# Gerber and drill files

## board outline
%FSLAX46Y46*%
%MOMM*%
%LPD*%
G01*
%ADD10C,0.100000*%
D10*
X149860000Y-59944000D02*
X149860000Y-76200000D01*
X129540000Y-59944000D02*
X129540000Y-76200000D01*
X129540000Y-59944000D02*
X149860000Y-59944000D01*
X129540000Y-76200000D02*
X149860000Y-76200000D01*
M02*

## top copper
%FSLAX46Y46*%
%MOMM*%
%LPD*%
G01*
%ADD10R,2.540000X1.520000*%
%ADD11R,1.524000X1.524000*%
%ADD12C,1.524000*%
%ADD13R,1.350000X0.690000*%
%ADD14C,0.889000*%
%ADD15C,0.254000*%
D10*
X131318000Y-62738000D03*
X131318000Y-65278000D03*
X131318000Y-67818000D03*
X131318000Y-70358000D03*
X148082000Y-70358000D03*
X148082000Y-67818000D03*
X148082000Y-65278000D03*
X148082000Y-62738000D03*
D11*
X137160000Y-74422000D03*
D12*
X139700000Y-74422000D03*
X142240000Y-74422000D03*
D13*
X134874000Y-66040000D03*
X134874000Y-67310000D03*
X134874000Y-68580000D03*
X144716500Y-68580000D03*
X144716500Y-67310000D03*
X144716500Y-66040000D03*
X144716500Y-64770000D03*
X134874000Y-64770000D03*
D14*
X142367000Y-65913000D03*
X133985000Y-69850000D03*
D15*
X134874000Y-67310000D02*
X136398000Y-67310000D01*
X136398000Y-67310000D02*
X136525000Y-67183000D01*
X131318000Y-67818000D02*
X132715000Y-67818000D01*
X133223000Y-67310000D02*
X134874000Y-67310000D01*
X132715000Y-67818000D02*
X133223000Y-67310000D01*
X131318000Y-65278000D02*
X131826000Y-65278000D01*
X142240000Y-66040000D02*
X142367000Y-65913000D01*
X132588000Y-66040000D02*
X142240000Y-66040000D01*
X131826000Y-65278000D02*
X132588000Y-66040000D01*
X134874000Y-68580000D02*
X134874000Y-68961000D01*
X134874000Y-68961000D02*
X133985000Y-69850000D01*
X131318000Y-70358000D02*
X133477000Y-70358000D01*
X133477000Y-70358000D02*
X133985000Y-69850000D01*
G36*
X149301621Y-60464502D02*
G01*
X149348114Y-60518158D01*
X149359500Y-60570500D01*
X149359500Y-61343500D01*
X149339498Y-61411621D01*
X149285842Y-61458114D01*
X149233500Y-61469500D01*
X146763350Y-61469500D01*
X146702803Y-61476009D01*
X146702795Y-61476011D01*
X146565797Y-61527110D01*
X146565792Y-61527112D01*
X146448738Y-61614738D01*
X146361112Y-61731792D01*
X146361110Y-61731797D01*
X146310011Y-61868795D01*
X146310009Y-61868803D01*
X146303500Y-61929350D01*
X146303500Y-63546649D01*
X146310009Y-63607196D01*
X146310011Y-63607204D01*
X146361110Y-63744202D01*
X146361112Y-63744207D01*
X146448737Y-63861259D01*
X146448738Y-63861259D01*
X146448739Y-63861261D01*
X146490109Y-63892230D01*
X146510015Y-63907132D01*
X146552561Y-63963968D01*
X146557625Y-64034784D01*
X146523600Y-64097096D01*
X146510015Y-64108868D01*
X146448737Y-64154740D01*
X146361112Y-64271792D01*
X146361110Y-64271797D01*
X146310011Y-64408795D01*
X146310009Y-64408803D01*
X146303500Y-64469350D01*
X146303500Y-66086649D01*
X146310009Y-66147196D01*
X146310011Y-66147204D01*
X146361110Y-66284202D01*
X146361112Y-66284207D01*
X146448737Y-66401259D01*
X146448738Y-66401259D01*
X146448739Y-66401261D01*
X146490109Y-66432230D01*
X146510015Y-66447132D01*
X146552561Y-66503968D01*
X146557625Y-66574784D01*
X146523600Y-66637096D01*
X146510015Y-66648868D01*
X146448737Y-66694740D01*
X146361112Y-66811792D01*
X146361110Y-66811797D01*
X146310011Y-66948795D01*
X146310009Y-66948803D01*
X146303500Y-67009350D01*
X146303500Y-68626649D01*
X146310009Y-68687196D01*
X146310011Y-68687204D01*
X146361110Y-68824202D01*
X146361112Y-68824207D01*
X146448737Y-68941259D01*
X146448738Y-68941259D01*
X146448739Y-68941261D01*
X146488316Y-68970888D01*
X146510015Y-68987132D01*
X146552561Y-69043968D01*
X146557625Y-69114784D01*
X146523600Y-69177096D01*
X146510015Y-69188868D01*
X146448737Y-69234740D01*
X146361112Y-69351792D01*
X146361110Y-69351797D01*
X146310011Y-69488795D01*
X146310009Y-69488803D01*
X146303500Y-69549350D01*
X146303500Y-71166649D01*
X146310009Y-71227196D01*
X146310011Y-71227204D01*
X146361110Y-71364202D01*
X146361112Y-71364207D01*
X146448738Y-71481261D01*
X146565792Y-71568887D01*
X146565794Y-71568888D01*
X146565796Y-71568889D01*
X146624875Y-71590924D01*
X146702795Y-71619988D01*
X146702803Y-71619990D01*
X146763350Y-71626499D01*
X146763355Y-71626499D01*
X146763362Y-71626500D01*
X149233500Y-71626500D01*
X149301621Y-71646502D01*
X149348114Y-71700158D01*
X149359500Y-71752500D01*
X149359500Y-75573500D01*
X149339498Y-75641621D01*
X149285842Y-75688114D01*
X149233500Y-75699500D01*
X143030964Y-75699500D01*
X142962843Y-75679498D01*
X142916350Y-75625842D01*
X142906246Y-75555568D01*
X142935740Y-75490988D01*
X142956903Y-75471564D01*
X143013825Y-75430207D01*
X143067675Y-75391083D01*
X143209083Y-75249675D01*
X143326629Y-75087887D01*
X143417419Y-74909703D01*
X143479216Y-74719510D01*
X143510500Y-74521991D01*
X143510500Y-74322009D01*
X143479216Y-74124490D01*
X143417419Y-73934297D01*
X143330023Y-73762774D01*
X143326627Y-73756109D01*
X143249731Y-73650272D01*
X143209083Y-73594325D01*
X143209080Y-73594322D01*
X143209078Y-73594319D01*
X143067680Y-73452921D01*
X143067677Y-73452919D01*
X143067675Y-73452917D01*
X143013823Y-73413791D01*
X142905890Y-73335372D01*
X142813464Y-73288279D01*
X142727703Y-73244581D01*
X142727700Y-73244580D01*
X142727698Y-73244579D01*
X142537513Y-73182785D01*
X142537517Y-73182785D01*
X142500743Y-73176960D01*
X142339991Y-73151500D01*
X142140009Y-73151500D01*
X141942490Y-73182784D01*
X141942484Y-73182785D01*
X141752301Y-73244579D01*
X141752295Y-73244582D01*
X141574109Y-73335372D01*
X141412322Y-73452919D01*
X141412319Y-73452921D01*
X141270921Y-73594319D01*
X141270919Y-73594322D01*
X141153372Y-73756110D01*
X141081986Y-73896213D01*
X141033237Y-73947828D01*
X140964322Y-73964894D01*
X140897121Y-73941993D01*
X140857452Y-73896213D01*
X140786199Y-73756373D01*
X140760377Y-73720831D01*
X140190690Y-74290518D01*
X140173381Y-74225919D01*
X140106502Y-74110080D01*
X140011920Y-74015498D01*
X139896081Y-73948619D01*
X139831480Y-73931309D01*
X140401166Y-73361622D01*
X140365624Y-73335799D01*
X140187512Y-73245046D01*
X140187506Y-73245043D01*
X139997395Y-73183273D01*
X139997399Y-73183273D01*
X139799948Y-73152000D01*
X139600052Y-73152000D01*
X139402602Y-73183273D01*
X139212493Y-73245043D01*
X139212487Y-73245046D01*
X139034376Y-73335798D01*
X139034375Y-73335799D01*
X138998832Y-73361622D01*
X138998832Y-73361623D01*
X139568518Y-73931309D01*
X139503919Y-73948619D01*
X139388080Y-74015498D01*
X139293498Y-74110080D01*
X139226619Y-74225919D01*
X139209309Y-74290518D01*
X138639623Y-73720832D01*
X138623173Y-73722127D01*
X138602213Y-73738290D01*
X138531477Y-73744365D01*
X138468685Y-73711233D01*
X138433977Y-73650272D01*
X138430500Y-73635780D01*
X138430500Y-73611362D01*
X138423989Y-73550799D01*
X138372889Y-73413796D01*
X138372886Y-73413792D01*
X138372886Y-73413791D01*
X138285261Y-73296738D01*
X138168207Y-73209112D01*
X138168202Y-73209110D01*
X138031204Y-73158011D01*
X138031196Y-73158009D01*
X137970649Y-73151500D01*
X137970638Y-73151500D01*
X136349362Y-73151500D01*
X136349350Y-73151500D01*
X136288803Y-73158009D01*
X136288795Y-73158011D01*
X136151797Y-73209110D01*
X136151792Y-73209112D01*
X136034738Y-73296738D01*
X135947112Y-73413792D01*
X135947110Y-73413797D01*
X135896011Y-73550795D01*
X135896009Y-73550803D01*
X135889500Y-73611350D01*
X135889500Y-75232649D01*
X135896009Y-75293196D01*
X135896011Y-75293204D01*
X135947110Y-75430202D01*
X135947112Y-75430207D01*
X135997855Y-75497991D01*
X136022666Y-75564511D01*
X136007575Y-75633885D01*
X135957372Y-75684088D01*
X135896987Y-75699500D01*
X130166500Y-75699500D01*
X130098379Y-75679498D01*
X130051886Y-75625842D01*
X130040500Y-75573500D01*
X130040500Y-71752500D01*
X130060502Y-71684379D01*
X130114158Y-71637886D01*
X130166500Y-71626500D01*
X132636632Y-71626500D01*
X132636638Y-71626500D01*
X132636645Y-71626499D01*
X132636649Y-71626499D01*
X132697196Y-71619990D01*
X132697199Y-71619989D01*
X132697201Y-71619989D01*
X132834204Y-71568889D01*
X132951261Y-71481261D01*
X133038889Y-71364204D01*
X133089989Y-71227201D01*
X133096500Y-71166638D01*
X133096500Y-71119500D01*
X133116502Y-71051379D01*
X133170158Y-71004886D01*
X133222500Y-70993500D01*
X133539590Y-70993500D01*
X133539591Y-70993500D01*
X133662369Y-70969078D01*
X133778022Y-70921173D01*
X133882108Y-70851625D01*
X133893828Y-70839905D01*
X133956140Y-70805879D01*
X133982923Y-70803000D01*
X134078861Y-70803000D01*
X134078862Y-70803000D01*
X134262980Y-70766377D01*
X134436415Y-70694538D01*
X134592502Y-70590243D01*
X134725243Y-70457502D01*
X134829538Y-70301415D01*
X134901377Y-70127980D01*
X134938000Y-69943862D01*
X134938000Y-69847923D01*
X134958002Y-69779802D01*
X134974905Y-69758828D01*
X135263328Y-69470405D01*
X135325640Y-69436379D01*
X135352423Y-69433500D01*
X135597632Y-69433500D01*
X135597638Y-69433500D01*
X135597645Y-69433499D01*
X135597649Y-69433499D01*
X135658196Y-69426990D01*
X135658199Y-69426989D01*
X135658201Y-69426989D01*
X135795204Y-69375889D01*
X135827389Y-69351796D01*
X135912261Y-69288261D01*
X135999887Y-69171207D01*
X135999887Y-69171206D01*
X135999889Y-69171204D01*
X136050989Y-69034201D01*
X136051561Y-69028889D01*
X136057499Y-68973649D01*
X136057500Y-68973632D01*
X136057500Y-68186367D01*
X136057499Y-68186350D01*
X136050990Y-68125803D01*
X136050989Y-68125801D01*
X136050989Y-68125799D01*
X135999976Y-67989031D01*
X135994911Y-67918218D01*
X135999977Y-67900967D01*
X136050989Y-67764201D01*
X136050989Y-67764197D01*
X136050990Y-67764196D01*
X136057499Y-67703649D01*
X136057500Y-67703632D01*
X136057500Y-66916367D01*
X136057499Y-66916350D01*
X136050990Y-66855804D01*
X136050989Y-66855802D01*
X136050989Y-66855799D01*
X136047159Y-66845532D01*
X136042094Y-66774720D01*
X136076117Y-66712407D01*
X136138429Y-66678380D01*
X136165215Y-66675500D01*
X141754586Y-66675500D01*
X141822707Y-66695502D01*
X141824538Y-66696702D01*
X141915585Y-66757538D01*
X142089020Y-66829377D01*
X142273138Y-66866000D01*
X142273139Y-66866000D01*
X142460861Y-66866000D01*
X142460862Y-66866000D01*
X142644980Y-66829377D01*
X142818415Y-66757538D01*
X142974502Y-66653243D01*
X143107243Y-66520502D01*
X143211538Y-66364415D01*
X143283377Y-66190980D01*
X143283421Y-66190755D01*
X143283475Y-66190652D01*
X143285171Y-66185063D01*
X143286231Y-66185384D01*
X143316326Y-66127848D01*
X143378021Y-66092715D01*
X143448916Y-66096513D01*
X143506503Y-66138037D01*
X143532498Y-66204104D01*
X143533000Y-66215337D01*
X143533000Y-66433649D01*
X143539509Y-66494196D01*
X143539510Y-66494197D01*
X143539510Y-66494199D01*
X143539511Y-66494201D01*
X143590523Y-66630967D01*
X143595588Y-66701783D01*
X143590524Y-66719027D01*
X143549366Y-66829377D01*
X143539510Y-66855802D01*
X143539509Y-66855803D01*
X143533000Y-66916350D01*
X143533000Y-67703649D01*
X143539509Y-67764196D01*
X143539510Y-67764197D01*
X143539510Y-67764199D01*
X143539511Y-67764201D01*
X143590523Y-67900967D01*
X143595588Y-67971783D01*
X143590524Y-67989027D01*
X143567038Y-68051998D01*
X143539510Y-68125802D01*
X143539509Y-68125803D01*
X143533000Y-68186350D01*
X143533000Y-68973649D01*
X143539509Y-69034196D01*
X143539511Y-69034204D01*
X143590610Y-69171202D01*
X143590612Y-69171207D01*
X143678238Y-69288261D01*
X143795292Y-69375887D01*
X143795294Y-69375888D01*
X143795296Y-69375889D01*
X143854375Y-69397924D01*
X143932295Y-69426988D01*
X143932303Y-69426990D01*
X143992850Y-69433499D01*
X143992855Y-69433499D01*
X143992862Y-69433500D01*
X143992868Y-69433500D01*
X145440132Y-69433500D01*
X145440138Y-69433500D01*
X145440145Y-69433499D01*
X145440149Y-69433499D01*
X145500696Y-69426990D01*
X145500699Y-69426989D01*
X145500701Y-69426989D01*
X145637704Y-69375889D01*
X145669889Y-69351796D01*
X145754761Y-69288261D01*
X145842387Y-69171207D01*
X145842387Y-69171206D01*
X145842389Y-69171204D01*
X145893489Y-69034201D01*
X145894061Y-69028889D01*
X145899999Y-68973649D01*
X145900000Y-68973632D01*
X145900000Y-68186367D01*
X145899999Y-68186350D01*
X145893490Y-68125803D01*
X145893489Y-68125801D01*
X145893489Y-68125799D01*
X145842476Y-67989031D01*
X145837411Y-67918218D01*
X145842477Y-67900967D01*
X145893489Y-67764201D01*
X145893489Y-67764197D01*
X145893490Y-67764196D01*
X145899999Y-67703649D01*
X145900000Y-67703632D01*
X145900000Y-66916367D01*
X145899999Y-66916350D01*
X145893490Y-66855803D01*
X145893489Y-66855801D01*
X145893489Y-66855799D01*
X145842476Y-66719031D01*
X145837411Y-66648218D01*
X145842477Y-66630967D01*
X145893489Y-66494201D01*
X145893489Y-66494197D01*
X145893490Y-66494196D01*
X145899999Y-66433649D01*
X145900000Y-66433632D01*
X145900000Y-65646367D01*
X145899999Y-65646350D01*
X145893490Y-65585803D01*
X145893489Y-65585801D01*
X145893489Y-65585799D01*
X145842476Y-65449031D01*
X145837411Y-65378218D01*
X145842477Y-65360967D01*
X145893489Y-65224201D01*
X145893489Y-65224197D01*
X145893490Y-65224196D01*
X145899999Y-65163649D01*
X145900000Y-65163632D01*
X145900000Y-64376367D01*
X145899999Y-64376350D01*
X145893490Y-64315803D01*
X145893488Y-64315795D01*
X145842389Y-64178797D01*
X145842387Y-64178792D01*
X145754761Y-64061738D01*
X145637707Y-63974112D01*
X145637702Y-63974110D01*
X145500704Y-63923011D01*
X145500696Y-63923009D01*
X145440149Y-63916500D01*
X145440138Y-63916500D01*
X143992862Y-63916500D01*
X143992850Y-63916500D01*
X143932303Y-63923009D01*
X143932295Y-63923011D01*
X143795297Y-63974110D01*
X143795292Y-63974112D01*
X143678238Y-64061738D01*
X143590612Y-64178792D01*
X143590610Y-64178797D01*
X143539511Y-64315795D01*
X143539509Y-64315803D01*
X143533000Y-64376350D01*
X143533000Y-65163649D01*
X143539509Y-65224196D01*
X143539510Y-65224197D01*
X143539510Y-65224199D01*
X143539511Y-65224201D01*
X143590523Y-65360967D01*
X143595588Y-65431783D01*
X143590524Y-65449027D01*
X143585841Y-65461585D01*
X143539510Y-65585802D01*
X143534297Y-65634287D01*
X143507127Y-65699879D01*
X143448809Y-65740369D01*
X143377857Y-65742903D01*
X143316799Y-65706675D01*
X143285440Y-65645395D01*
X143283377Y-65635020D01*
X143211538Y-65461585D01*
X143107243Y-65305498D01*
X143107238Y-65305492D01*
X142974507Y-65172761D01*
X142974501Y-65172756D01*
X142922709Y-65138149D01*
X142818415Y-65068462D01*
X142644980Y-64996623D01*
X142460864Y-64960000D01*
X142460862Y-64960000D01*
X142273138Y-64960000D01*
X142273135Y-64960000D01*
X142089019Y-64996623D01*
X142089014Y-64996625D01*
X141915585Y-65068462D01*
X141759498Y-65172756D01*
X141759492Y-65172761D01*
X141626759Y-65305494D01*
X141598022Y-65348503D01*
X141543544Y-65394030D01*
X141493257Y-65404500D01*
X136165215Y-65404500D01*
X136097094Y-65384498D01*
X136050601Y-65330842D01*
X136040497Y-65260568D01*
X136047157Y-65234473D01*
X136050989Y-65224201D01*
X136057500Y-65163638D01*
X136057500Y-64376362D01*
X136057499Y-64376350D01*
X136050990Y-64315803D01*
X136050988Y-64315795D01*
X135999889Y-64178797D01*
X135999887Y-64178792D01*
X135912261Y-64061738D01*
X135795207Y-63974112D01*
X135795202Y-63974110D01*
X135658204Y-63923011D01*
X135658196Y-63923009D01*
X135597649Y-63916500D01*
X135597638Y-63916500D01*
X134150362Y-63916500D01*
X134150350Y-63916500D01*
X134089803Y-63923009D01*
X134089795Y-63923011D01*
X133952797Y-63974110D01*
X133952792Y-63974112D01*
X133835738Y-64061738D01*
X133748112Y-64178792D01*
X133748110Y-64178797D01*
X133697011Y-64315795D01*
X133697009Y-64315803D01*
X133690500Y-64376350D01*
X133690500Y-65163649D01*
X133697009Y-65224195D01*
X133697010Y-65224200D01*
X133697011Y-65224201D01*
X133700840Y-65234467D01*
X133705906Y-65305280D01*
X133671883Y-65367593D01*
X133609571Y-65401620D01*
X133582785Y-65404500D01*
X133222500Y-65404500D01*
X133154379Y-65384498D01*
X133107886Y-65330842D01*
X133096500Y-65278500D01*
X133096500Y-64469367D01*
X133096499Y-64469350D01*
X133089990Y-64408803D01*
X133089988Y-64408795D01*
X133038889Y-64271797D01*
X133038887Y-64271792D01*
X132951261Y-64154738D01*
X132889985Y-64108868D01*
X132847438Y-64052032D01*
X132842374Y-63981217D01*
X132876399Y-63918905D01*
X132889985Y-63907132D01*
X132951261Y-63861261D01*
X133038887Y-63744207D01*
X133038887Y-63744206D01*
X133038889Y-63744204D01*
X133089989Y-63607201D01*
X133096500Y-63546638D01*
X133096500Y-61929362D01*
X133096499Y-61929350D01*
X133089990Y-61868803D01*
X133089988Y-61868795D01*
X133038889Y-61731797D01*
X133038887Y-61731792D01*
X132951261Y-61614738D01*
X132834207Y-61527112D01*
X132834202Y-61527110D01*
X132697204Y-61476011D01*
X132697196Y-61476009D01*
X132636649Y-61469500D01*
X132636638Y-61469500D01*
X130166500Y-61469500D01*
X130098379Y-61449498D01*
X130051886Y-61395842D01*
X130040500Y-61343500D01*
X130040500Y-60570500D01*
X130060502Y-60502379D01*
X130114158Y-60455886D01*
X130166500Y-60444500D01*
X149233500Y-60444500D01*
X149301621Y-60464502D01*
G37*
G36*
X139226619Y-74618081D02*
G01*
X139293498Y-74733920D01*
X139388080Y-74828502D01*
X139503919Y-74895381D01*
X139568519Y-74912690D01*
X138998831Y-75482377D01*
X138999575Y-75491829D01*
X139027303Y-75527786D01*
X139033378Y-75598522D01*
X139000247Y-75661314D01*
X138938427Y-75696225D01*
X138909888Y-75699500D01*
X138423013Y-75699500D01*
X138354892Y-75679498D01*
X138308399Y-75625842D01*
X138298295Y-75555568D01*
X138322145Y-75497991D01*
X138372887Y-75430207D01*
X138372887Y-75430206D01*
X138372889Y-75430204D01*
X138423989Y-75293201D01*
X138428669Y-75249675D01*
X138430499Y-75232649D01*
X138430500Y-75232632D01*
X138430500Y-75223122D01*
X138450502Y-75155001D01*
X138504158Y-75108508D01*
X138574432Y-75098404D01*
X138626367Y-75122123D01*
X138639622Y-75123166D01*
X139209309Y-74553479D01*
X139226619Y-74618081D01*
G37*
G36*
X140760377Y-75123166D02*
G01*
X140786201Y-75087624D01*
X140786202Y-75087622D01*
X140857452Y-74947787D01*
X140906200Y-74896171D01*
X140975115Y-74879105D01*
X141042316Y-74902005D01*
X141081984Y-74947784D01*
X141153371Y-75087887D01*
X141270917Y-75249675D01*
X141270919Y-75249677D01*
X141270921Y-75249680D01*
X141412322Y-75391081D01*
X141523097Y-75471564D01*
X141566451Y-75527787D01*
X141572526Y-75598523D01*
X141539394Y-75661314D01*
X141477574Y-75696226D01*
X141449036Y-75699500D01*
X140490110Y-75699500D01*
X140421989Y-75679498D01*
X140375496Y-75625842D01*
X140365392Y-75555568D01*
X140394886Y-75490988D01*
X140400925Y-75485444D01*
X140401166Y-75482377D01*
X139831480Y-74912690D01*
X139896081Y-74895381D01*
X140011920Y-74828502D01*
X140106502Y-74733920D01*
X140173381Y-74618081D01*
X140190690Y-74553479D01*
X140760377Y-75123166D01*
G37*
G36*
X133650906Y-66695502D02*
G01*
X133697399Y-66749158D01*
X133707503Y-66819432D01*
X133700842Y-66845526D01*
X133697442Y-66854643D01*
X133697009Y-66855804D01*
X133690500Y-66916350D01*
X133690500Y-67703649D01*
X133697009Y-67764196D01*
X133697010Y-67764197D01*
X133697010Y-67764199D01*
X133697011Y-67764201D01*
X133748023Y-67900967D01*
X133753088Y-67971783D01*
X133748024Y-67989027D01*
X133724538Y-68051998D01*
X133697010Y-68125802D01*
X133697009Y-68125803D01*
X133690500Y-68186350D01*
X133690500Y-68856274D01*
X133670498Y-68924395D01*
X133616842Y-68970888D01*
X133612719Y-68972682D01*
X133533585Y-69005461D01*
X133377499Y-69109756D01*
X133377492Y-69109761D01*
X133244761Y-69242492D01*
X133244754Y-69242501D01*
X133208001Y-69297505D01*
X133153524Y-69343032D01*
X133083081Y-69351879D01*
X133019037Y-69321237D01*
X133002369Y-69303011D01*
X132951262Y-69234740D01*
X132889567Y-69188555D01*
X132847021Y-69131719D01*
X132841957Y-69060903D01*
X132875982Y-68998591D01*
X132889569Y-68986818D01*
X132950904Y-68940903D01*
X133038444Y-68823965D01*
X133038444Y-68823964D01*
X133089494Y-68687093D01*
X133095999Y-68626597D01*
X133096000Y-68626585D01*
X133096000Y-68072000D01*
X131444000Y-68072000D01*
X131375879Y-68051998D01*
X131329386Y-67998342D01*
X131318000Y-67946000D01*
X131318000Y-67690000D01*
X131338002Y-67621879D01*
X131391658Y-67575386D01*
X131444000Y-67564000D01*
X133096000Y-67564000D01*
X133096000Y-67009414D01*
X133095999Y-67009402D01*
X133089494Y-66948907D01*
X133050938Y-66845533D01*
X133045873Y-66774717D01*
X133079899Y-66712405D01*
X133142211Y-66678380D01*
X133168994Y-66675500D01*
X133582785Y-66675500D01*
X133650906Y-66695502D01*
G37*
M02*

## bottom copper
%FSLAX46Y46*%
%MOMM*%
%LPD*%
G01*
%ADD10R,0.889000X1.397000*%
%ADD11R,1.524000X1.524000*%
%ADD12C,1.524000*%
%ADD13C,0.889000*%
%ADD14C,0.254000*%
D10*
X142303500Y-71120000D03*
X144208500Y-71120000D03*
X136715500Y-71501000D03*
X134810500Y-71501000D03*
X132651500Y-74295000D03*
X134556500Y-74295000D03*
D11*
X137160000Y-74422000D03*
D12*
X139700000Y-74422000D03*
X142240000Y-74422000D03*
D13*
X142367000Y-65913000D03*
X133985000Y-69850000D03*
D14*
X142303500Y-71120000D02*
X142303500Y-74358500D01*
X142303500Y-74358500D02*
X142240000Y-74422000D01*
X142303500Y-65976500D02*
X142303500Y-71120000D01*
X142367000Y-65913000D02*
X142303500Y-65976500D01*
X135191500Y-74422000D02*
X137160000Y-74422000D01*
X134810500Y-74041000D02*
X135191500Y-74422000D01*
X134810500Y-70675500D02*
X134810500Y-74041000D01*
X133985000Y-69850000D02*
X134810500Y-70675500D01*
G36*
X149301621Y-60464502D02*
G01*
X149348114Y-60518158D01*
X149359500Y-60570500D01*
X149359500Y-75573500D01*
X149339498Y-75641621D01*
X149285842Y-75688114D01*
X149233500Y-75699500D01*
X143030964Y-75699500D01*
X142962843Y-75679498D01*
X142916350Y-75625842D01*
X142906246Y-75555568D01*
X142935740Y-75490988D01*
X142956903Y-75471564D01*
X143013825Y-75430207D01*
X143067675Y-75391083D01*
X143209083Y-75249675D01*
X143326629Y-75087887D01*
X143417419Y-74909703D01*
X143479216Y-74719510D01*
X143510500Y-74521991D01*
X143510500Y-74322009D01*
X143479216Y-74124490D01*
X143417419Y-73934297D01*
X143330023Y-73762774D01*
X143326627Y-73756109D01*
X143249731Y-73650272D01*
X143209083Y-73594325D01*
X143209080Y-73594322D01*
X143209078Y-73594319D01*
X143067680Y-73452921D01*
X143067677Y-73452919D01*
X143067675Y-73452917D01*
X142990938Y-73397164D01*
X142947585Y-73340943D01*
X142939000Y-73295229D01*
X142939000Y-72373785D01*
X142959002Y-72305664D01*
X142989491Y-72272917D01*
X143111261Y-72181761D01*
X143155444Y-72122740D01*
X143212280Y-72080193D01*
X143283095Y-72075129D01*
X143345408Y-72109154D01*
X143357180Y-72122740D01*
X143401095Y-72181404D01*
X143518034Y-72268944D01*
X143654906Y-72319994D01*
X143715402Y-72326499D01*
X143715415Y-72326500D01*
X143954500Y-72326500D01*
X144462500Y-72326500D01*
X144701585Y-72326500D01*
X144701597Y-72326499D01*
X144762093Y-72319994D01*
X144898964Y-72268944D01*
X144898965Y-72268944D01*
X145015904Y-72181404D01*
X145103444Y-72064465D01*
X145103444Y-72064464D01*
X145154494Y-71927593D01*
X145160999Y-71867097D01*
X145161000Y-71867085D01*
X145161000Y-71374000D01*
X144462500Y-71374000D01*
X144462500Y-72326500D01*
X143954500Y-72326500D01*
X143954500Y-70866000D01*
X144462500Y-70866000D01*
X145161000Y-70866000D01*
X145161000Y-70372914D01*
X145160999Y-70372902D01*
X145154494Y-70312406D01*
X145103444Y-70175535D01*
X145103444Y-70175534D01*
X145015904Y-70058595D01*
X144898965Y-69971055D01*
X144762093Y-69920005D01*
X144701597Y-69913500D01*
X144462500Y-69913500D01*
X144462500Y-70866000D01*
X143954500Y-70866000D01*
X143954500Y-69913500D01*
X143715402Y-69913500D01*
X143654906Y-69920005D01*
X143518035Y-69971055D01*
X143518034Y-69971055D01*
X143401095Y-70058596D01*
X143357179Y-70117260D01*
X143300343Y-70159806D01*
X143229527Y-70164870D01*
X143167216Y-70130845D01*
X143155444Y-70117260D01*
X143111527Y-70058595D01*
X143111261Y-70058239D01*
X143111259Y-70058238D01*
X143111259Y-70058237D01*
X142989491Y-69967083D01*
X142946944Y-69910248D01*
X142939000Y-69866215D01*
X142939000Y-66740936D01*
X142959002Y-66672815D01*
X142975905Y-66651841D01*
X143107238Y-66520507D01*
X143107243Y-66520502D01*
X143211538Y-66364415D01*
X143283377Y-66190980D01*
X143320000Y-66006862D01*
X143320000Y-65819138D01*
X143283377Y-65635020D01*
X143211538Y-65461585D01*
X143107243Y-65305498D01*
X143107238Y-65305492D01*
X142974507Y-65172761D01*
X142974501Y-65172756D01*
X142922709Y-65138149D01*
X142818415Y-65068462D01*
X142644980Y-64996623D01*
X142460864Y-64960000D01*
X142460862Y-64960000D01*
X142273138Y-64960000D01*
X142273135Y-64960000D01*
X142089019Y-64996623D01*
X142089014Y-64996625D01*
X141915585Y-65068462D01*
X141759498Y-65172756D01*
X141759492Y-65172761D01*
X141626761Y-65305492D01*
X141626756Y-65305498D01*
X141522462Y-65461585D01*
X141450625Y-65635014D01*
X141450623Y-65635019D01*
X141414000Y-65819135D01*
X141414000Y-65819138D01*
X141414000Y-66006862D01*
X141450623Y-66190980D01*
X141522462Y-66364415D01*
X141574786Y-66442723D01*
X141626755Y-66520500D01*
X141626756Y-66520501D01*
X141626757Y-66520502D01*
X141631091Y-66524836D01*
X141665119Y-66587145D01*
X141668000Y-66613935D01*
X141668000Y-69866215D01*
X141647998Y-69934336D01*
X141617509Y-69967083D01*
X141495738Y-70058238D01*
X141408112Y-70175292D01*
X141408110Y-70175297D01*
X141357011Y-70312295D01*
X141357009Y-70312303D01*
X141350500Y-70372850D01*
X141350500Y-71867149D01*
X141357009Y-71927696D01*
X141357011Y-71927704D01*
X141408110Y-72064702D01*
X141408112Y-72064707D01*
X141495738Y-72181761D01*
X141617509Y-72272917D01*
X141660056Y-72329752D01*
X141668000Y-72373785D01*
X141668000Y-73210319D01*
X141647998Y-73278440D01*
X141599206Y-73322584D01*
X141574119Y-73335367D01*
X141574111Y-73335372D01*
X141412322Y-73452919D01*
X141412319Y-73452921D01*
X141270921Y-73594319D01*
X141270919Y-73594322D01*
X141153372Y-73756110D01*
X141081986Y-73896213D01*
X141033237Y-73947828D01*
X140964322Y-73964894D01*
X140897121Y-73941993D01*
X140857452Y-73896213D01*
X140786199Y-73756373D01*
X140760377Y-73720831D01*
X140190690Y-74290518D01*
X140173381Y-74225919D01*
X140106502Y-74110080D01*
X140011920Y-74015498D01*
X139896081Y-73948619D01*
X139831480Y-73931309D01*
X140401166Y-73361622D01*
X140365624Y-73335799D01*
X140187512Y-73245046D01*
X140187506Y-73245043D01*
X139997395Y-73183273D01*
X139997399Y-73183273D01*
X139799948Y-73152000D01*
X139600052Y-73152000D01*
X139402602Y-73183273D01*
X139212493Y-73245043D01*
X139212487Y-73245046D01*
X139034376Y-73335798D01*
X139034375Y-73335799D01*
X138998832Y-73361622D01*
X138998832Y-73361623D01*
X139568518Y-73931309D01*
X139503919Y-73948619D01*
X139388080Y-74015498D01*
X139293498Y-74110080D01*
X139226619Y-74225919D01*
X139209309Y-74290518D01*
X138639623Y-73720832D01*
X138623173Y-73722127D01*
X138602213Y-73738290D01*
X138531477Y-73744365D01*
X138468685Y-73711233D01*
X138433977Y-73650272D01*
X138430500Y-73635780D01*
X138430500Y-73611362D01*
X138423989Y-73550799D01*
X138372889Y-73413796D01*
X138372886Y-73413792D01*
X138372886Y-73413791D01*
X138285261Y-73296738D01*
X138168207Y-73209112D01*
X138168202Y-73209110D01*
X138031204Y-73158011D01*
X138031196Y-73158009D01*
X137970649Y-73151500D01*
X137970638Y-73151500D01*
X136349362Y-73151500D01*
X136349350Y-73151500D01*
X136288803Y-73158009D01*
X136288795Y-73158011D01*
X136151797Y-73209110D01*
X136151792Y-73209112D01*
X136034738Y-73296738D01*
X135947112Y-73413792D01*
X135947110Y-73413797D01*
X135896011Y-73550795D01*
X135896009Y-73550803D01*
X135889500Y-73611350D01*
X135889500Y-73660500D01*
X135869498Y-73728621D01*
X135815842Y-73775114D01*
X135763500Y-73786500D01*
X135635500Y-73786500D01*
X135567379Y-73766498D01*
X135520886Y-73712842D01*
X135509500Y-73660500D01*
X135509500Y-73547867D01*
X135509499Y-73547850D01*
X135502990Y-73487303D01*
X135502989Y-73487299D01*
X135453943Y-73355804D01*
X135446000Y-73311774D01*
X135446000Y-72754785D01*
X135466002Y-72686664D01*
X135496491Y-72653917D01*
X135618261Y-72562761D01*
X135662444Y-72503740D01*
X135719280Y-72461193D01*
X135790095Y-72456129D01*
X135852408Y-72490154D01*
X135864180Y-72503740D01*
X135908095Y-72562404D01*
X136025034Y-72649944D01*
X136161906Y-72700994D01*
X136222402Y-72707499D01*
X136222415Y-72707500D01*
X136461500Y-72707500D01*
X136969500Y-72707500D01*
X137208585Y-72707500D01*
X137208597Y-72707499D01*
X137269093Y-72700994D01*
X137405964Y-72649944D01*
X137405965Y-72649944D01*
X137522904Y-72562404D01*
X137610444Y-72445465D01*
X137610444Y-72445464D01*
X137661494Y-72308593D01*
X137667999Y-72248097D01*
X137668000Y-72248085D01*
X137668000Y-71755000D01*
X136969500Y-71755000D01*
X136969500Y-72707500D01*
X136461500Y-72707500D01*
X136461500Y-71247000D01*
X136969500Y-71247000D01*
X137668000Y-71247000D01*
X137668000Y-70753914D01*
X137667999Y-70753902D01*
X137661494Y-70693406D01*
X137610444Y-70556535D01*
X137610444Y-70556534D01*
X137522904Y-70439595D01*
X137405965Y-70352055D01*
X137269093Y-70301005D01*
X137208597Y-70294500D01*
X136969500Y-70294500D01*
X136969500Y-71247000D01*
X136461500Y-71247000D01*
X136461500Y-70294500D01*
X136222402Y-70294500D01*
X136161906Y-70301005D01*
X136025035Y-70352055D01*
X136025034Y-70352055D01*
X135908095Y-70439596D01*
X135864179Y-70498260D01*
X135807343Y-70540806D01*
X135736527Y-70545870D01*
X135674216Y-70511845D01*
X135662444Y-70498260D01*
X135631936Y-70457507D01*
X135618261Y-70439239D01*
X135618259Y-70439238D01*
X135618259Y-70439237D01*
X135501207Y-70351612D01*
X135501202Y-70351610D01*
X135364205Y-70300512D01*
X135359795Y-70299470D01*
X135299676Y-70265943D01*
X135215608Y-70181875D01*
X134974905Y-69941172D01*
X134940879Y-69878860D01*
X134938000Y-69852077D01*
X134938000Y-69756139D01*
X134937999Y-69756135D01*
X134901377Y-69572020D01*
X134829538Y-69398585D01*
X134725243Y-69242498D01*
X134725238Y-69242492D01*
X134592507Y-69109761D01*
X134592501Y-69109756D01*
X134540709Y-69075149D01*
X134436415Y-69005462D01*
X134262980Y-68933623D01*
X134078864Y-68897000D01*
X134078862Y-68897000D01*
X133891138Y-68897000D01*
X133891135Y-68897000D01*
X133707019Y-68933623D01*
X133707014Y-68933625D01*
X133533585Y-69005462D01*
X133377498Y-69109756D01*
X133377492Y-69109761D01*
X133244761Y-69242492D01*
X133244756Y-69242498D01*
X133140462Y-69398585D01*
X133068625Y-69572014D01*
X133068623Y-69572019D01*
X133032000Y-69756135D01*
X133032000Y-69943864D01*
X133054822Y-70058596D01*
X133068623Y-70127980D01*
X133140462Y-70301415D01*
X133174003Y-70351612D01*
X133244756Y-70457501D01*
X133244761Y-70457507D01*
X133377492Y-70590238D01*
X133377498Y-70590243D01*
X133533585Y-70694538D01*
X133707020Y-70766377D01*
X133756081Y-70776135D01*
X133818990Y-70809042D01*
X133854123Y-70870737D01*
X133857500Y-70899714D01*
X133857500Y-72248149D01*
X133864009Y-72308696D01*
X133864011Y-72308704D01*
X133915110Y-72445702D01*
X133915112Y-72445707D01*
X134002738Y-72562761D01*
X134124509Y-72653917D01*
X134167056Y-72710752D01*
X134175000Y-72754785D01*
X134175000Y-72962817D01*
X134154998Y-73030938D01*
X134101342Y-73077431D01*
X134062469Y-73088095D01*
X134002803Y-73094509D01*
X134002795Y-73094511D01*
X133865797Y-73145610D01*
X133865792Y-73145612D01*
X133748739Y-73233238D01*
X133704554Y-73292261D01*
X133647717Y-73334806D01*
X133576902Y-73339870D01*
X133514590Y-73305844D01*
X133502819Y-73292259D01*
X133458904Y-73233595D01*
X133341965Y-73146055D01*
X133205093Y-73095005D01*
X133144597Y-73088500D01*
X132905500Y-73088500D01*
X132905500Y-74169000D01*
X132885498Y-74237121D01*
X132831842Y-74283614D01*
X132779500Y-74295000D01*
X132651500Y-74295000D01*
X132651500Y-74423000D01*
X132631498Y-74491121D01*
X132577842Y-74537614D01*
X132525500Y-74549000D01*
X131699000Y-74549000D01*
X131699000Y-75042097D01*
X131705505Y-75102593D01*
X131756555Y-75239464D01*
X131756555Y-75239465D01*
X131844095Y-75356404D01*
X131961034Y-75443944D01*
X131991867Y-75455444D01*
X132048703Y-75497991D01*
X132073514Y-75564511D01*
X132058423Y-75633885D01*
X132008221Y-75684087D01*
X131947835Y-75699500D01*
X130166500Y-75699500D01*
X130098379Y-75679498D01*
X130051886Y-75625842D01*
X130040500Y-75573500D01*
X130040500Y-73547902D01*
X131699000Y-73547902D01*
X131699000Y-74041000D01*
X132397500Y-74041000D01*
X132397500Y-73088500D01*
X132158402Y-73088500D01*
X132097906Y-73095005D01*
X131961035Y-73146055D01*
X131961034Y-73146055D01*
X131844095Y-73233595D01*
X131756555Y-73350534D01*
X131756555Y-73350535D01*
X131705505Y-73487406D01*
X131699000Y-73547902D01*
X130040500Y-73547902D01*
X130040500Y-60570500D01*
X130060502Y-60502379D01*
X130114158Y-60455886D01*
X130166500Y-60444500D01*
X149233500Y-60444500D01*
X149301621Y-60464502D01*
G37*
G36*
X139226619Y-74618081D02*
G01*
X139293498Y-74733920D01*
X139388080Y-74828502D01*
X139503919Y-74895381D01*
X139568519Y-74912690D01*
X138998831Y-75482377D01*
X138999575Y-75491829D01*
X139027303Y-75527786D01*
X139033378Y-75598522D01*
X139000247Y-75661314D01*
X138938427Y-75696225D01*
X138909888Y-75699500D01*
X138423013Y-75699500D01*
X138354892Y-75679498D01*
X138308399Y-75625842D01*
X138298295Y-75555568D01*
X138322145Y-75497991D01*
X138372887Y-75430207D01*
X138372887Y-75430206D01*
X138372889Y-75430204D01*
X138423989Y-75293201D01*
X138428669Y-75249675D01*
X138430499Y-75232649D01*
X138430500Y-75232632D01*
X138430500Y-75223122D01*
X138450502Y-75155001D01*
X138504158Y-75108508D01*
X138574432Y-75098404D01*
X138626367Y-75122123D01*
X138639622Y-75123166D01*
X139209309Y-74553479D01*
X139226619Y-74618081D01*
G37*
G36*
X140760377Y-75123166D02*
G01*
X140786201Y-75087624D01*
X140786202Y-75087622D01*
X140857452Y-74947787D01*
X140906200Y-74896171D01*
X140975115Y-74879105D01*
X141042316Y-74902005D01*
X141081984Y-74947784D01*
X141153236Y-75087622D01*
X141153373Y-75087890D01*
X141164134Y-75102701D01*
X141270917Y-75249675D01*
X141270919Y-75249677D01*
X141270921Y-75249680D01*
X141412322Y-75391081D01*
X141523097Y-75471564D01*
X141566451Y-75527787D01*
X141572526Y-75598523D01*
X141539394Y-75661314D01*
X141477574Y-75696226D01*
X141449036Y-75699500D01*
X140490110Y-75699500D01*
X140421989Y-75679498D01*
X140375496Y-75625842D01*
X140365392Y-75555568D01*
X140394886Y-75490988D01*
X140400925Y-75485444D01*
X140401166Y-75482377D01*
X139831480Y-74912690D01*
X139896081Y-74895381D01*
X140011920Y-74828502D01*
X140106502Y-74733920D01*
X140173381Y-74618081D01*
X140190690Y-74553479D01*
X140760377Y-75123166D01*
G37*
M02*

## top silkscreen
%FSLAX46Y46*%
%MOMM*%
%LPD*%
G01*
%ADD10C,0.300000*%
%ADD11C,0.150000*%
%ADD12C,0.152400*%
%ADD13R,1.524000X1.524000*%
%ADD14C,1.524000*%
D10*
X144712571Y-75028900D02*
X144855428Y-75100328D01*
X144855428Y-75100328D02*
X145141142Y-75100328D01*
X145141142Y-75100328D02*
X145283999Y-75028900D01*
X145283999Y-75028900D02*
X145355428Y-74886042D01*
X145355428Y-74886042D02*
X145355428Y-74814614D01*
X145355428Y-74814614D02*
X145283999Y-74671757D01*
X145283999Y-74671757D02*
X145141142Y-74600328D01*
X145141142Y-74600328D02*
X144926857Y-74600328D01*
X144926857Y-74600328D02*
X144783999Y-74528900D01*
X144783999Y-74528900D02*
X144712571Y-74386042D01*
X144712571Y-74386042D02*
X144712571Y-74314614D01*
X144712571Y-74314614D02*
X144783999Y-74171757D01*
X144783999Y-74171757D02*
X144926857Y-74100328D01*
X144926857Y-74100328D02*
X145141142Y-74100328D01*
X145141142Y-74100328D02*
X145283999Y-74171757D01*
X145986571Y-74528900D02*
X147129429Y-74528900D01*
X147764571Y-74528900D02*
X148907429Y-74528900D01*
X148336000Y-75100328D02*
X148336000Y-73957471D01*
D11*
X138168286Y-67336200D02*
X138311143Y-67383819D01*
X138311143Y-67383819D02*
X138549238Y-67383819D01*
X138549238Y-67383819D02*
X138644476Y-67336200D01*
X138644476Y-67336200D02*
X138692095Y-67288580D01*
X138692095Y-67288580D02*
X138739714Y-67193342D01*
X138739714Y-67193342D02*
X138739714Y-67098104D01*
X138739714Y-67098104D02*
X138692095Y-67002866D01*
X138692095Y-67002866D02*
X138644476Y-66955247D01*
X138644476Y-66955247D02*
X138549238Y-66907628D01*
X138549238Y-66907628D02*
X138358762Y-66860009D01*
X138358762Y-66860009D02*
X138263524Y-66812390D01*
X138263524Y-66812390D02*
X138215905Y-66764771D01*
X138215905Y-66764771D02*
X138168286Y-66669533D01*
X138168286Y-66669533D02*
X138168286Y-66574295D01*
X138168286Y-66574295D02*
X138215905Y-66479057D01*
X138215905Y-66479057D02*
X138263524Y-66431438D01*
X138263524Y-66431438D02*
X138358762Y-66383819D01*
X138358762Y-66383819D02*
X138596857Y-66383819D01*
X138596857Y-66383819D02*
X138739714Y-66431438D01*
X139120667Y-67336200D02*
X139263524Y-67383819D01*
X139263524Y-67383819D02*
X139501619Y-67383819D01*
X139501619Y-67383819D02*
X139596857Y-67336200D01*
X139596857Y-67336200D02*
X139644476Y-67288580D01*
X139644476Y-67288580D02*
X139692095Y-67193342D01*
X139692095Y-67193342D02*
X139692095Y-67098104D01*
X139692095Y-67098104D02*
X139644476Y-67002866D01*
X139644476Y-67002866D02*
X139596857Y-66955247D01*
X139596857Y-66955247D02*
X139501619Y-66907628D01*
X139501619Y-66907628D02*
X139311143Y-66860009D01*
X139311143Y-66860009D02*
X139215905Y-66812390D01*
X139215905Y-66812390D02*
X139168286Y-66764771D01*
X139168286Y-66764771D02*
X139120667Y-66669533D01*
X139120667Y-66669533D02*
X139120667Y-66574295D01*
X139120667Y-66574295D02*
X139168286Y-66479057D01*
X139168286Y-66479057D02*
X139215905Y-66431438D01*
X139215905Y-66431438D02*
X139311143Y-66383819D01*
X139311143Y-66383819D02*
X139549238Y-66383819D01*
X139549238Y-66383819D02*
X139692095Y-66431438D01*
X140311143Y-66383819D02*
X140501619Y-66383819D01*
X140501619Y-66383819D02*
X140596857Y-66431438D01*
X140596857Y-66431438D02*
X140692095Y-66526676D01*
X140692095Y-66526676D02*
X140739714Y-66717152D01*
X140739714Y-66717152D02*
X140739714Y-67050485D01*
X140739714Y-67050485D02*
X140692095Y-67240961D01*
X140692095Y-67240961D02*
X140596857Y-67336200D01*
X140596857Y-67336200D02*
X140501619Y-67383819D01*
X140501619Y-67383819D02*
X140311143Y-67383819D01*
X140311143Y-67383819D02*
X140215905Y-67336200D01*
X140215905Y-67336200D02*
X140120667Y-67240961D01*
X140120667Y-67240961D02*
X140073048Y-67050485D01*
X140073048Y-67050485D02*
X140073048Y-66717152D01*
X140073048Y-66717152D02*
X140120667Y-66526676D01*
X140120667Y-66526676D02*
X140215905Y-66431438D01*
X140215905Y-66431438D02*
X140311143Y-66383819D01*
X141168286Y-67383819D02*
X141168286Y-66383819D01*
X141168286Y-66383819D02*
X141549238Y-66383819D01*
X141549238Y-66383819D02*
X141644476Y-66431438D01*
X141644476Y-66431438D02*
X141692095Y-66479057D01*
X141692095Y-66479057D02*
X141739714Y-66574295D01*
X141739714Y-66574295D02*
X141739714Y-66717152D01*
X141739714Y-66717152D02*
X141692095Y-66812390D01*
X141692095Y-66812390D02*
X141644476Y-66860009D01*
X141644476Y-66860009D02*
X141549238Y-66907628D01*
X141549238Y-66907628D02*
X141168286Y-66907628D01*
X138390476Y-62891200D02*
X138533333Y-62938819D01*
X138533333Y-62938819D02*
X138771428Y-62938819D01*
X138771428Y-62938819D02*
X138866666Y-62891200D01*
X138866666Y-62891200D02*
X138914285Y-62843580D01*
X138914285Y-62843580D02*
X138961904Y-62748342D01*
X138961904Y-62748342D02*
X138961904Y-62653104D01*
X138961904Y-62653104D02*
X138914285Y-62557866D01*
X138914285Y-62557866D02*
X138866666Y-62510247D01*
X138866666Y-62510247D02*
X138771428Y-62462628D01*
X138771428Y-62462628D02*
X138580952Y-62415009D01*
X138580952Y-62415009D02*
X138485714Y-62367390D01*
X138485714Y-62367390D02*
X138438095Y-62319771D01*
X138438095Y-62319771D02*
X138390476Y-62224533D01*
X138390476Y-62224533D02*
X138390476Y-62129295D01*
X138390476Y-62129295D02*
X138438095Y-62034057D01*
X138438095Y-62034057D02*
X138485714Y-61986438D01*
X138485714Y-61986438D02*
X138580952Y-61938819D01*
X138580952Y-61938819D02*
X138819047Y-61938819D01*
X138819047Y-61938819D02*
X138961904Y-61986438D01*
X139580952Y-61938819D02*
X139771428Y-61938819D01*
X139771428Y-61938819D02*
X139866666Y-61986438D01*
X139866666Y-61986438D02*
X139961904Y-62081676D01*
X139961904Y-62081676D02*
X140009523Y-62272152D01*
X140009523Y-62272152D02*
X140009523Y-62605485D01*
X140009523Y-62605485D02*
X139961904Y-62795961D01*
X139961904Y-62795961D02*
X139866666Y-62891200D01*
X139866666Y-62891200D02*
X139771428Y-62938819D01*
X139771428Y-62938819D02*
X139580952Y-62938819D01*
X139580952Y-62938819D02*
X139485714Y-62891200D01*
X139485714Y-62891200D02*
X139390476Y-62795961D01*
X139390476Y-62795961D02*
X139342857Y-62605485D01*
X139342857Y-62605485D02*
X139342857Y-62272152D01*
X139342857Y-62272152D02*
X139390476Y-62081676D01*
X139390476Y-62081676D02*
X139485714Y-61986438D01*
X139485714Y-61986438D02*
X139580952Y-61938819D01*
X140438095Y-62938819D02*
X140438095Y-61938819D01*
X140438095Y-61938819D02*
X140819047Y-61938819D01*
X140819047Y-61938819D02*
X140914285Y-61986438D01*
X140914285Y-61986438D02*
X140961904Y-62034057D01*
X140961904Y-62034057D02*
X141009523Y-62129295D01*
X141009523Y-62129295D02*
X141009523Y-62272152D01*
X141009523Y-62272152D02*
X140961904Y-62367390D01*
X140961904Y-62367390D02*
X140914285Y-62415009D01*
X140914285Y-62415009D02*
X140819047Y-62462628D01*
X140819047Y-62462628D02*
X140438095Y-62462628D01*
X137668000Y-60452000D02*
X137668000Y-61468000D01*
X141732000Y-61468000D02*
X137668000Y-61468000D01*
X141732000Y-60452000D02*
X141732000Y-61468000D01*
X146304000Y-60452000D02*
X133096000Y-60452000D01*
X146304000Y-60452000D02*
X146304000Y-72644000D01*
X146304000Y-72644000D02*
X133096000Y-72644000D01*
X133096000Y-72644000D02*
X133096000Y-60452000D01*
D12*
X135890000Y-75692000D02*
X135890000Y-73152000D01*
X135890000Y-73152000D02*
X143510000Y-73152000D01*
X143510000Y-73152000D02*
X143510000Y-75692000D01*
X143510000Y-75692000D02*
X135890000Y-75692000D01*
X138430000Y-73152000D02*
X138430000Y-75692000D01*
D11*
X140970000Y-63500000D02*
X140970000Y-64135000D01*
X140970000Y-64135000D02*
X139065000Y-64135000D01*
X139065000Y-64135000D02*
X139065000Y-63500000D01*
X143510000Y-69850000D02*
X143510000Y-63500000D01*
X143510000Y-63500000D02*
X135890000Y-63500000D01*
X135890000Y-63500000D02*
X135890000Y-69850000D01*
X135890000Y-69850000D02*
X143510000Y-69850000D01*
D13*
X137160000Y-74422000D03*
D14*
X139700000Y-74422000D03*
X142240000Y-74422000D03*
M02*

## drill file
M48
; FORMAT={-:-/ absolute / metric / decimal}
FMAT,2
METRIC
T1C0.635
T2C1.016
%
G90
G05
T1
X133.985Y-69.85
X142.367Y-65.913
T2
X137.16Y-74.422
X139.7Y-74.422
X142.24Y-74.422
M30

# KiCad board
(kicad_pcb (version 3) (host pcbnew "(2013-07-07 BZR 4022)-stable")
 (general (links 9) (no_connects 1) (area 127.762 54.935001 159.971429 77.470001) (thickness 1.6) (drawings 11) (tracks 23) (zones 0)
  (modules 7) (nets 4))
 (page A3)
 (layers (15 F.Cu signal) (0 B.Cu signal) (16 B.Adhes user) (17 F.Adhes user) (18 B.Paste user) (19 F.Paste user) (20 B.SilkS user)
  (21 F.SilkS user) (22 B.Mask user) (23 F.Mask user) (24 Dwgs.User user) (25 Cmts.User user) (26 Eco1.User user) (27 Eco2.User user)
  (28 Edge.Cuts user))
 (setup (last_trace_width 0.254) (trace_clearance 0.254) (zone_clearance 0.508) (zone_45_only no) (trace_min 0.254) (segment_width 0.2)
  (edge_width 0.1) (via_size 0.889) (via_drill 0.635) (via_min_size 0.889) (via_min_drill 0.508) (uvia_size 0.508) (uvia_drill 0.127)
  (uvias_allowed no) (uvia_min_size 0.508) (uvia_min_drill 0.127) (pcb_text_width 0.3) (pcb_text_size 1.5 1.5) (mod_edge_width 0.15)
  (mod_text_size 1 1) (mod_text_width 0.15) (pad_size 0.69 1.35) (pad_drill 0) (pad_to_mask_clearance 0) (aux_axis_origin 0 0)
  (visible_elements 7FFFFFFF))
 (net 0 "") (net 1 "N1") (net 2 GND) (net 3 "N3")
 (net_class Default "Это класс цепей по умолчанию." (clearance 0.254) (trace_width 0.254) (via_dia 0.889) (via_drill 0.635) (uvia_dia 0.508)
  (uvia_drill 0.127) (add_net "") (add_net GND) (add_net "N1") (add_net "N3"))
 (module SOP (layer F.Cu) (at 139.7 66.548)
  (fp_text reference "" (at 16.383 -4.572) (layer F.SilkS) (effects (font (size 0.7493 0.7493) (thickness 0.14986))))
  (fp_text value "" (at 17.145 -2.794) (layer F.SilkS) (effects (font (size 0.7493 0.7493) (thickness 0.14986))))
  (fp_line (start -2.032 -6.096) (end -2.032 -5.08) (layer F.SilkS) (width 0.15))
  (fp_line (start 2.032 -5.08) (end -2.032 -5.08) (layer F.SilkS) (width 0.15))
  (fp_line (start 2.032 -6.096) (end 2.032 -5.08) (layer F.SilkS) (width 0.15))
  (fp_line (start 6.604 -6.096) (end -6.604 -6.096) (layer F.SilkS) (width 0.15))
  (fp_line (start 6.604 -6.096) (end 6.604 6.096) (layer F.SilkS) (width 0.15))
  (fp_line (start 6.604 6.096) (end -6.604 6.096) (layer F.SilkS) (width 0.15))
  (fp_line (start -6.604 6.096) (end -6.604 -6.096) (layer F.SilkS) (width 0.15))
  (pad 1 smd rect (at -8.382 -3.81 270) (size 1.52 2.54) (layers F.Cu F.Paste F.Mask))
  (pad 2 smd rect (at -8.382 -1.27 270) (size 1.52 2.54) (layers F.Cu F.Paste F.Mask) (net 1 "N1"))
  (pad 3 smd rect (at -8.382 1.27 270) (size 1.52 2.54) (layers F.Cu F.Paste F.Mask) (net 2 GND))
  (pad 4 smd rect (at -8.382 3.81 270) (size 1.52 2.54) (layers F.Cu F.Paste F.Mask) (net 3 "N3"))
  (pad 5 smd rect (at 8.382 3.81 270) (size 1.52 2.54) (layers F.Cu F.Paste F.Mask))
  (pad 6 smd rect (at 8.382 1.27 270) (size 1.52 2.54) (layers F.Cu F.Paste F.Mask))
  (pad 7 smd rect (at 8.382 -1.27 270) (size 1.52 2.54) (layers F.Cu F.Paste F.Mask))
  (pad 8 smd rect (at 8.382 -3.81 270) (size 1.52 2.54) (layers F.Cu F.Paste F.Mask)))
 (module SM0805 (layer B.Cu) (at 143.256 71.12)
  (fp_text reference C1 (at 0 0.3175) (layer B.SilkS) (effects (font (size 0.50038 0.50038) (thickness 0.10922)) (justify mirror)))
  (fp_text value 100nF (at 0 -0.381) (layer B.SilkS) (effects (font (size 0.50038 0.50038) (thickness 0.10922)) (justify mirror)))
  (pad 1 smd rect (at -0.9525 0) (size 0.889 1.397) (layers B.Cu B.Paste B.Mask) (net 1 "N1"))
  (pad 2 smd rect (at 0.9525 0) (size 0.889 1.397) (layers B.Cu B.Paste B.Mask) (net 2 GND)))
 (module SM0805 (layer B.Cu) (at 135.763 71.501 180)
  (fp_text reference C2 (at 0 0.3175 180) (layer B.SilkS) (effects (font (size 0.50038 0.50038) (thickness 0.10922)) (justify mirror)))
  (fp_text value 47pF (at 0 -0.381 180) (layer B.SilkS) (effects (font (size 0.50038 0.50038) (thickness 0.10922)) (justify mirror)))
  (pad 1 smd rect (at -0.9525 0 180) (size 0.889 1.397) (layers B.Cu B.Paste B.Mask) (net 2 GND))
  (pad 2 smd rect (at 0.9525 0 180) (size 0.889 1.397) (layers B.Cu B.Paste B.Mask) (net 3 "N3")))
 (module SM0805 (layer B.Cu) (at 133.604 74.295)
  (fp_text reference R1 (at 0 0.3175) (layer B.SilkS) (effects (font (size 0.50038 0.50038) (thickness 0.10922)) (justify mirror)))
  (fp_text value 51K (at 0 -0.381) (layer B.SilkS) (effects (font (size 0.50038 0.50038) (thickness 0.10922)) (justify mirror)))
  (pad 1 smd rect (at -0.9525 0) (size 0.889 1.397) (layers B.Cu B.Paste B.Mask) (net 2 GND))
  (pad 2 smd rect (at 0.9525 0) (size 0.889 1.397) (layers B.Cu B.Paste B.Mask) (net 3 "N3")))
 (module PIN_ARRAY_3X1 (layer F.Cu) (at 139.7 74.422)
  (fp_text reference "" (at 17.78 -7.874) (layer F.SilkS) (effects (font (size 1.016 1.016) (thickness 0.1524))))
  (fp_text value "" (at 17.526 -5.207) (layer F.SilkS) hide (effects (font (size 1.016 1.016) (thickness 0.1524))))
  (fp_line (start -3.81 1.27) (end -3.81 -1.27) (layer F.SilkS) (width 0.1524))
  (fp_line (start -3.81 -1.27) (end 3.81 -1.27) (layer F.SilkS) (width 0.1524))
  (fp_line (start 3.81 -1.27) (end 3.81 1.27) (layer F.SilkS) (width 0.1524))
  (fp_line (start 3.81 1.27) (end -3.81 1.27) (layer F.SilkS) (width 0.1524))
  (fp_line (start -1.27 -1.27) (end -1.27 1.27) (layer F.SilkS) (width 0.1524))
  (pad 1 thru_hole rect (at -2.54 0) (size 1.524 1.524) (drill 1.016) (layers *.Cu *.Mask F.SilkS) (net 3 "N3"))
  (pad 2 thru_hole circle (at 0 0) (size 1.524 1.524) (drill 1.016) (layers *.Cu *.Mask F.SilkS) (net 2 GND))
  (pad 3 thru_hole circle (at 2.54 0) (size 1.524 1.524) (drill 1.016) (layers *.Cu *.Mask F.SilkS) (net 1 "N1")))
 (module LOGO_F (layer B.Cu) (at 146.177 66.675)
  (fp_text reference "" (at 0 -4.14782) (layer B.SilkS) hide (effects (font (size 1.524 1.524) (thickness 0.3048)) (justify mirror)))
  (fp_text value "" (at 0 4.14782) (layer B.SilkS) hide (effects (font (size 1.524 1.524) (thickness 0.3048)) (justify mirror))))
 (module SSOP (layer F.Cu) (at 139.7 66.675)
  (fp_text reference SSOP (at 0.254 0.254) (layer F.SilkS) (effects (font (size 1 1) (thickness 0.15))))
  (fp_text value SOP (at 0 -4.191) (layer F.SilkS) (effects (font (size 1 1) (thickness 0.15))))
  (fp_line (start 1.27 -3.175) (end 1.27 -2.54) (layer F.SilkS) (width 0.15))
  (fp_line (start 1.27 -2.54) (end -0.635 -2.54) (layer F.SilkS) (width 0.15))
  (fp_line (start -0.635 -2.54) (end -0.635 -3.175) (layer F.SilkS) (width 0.15))
  (fp_line (start 3.81 3.175) (end 3.81 -3.175) (layer F.SilkS) (width 0.15))
  (fp_line (start 3.81 -3.175) (end -3.81 -3.175) (layer F.SilkS) (width 0.15))
  (fp_line (start -3.81 -3.175) (end -3.81 3.175) (layer F.SilkS) (width 0.15))
  (fp_line (start -3.81 3.175) (end 3.81 3.175) (layer F.SilkS) (width 0.15))
  (pad 2 smd rect (at -4.826 -0.635 270) (size 0.69 1.35) (layers F.Cu F.Paste F.Mask))
  (pad 3 smd rect (at -4.826 0.635 270) (size 0.69 1.35) (layers F.Cu F.Paste F.Mask))
  (pad 4 smd rect (at -4.826 1.905 270) (size 0.69 1.35) (layers F.Cu F.Paste F.Mask))
  (pad 5 smd rect (at 5.0165 1.905 270) (size 0.69 1.35) (layers F.Cu F.Paste F.Mask))
  (pad 6 smd rect (at 5.0165 0.635 270) (size 0.69 1.35) (layers F.Cu F.Paste F.Mask))
  (pad 7 smd rect (at 5.0165 -0.635 270) (size 0.69 1.35) (layers F.Cu F.Paste F.Mask))
  (pad 8 smd rect (at 5.0165 -1.905 270) (size 0.69 1.35) (layers F.Cu F.Paste F.Mask))
  (pad 1 smd rect (at -4.826 -1.905 270) (size 0.69 1.35) (layers F.Cu F.Paste F.Mask)))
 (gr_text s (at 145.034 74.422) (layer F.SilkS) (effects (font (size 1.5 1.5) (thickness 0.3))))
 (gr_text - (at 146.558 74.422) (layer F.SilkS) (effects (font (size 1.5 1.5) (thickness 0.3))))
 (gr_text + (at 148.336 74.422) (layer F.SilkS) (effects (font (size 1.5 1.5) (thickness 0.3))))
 (gr_line (start 149.86 59.944) (end 149.86 76.2) (angle 90) (layer Edge.Cuts) (width 0.1))
 (gr_line (start 129.54 59.944) (end 129.54 76.2) (angle 90) (layer Edge.Cuts) (width 0.1))
 (gr_line (start 129.54 59.944) (end 149.86 59.944) (angle 90) (layer Edge.Cuts) (width 0.1))
 (gr_line (start 129.54 76.2) (end 149.86 76.2) (angle 90) (layer Edge.Cuts) (width 0.1))
 (segment (start 134.874 67.31) (end 136.398 67.31) (width 0.254) (layer F.Cu) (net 2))
 (segment (start 136.398 67.31) (end 136.525 67.183) (width 0.254) (layer F.Cu) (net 2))
 (segment (start 131.318 67.818) (end 132.715 67.818) (width 0.254) (layer F.Cu) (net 2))
 (segment (start 133.223 67.31) (end 134.874 67.31) (width 0.254) (layer F.Cu) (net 2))
 (segment (start 132.715 67.818) (end 133.223 67.31) (width 0.254) (layer F.Cu) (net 2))
 (segment (start 142.3035 71.12) (end 142.3035 74.3585) (width 0.254) (layer B.Cu) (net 1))
 (segment (start 142.3035 74.3585) (end 142.24 74.422) (width 0.254) (layer B.Cu) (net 1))
 (segment (start 131.318 65.278) (end 131.826 65.278) (width 0.254) (layer F.Cu) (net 1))
 (segment (start 142.3035 65.9765) (end 142.3035 71.12) (width 0.254) (layer B.Cu) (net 1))
 (segment (start 142.367 65.913) (end 142.3035 65.9765) (width 0.254) (layer B.Cu) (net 1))
 (via (at 142.367 65.913) (size 0.889) (layers F.Cu B.Cu) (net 1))
 (segment (start 142.24 66.04) (end 142.367 65.913) (width 0.254) (layer F.Cu) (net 1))
 (segment (start 132.588 66.04) (end 142.24 66.04) (width 0.254) (layer F.Cu) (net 1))
 (segment (start 131.826 65.278) (end 132.588 66.04) (width 0.254) (layer F.Cu) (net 1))
 (segment (start 134.874 68.58) (end 134.874 68.961) (width 0.254) (layer F.Cu) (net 3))
 (segment (start 134.874 68.961) (end 133.985 69.85) (width 0.254) (layer F.Cu) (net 3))
 (segment (start 131.318 70.358) (end 133.477 70.358) (width 0.254) (layer F.Cu) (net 3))
 (segment (start 135.1915 74.422) (end 137.16 74.422) (width 0.254) (layer B.Cu) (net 3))
 (segment (start 134.8105 74.041) (end 135.1915 74.422) (width 0.254) (layer B.Cu) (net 3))
 (segment (start 134.8105 70.6755) (end 134.8105 74.041) (width 0.254) (layer B.Cu) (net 3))
 (segment (start 133.985 69.85) (end 134.8105 70.6755) (width 0.254) (layer B.Cu) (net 3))
 (via (at 133.985 69.85) (size 0.889) (layers F.Cu B.Cu) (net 3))
 (segment (start 133.477 70.358) (end 133.985 69.85) (width 0.254) (layer F.Cu) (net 3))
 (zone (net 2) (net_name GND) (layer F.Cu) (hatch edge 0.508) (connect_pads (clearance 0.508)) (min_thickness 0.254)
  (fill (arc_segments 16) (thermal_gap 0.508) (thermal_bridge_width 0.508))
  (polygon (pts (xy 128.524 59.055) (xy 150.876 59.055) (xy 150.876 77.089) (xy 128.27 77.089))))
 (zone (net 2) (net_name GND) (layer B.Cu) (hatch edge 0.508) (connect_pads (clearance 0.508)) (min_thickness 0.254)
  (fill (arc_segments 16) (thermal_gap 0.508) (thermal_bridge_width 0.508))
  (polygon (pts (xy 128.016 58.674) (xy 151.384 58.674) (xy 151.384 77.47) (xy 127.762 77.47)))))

